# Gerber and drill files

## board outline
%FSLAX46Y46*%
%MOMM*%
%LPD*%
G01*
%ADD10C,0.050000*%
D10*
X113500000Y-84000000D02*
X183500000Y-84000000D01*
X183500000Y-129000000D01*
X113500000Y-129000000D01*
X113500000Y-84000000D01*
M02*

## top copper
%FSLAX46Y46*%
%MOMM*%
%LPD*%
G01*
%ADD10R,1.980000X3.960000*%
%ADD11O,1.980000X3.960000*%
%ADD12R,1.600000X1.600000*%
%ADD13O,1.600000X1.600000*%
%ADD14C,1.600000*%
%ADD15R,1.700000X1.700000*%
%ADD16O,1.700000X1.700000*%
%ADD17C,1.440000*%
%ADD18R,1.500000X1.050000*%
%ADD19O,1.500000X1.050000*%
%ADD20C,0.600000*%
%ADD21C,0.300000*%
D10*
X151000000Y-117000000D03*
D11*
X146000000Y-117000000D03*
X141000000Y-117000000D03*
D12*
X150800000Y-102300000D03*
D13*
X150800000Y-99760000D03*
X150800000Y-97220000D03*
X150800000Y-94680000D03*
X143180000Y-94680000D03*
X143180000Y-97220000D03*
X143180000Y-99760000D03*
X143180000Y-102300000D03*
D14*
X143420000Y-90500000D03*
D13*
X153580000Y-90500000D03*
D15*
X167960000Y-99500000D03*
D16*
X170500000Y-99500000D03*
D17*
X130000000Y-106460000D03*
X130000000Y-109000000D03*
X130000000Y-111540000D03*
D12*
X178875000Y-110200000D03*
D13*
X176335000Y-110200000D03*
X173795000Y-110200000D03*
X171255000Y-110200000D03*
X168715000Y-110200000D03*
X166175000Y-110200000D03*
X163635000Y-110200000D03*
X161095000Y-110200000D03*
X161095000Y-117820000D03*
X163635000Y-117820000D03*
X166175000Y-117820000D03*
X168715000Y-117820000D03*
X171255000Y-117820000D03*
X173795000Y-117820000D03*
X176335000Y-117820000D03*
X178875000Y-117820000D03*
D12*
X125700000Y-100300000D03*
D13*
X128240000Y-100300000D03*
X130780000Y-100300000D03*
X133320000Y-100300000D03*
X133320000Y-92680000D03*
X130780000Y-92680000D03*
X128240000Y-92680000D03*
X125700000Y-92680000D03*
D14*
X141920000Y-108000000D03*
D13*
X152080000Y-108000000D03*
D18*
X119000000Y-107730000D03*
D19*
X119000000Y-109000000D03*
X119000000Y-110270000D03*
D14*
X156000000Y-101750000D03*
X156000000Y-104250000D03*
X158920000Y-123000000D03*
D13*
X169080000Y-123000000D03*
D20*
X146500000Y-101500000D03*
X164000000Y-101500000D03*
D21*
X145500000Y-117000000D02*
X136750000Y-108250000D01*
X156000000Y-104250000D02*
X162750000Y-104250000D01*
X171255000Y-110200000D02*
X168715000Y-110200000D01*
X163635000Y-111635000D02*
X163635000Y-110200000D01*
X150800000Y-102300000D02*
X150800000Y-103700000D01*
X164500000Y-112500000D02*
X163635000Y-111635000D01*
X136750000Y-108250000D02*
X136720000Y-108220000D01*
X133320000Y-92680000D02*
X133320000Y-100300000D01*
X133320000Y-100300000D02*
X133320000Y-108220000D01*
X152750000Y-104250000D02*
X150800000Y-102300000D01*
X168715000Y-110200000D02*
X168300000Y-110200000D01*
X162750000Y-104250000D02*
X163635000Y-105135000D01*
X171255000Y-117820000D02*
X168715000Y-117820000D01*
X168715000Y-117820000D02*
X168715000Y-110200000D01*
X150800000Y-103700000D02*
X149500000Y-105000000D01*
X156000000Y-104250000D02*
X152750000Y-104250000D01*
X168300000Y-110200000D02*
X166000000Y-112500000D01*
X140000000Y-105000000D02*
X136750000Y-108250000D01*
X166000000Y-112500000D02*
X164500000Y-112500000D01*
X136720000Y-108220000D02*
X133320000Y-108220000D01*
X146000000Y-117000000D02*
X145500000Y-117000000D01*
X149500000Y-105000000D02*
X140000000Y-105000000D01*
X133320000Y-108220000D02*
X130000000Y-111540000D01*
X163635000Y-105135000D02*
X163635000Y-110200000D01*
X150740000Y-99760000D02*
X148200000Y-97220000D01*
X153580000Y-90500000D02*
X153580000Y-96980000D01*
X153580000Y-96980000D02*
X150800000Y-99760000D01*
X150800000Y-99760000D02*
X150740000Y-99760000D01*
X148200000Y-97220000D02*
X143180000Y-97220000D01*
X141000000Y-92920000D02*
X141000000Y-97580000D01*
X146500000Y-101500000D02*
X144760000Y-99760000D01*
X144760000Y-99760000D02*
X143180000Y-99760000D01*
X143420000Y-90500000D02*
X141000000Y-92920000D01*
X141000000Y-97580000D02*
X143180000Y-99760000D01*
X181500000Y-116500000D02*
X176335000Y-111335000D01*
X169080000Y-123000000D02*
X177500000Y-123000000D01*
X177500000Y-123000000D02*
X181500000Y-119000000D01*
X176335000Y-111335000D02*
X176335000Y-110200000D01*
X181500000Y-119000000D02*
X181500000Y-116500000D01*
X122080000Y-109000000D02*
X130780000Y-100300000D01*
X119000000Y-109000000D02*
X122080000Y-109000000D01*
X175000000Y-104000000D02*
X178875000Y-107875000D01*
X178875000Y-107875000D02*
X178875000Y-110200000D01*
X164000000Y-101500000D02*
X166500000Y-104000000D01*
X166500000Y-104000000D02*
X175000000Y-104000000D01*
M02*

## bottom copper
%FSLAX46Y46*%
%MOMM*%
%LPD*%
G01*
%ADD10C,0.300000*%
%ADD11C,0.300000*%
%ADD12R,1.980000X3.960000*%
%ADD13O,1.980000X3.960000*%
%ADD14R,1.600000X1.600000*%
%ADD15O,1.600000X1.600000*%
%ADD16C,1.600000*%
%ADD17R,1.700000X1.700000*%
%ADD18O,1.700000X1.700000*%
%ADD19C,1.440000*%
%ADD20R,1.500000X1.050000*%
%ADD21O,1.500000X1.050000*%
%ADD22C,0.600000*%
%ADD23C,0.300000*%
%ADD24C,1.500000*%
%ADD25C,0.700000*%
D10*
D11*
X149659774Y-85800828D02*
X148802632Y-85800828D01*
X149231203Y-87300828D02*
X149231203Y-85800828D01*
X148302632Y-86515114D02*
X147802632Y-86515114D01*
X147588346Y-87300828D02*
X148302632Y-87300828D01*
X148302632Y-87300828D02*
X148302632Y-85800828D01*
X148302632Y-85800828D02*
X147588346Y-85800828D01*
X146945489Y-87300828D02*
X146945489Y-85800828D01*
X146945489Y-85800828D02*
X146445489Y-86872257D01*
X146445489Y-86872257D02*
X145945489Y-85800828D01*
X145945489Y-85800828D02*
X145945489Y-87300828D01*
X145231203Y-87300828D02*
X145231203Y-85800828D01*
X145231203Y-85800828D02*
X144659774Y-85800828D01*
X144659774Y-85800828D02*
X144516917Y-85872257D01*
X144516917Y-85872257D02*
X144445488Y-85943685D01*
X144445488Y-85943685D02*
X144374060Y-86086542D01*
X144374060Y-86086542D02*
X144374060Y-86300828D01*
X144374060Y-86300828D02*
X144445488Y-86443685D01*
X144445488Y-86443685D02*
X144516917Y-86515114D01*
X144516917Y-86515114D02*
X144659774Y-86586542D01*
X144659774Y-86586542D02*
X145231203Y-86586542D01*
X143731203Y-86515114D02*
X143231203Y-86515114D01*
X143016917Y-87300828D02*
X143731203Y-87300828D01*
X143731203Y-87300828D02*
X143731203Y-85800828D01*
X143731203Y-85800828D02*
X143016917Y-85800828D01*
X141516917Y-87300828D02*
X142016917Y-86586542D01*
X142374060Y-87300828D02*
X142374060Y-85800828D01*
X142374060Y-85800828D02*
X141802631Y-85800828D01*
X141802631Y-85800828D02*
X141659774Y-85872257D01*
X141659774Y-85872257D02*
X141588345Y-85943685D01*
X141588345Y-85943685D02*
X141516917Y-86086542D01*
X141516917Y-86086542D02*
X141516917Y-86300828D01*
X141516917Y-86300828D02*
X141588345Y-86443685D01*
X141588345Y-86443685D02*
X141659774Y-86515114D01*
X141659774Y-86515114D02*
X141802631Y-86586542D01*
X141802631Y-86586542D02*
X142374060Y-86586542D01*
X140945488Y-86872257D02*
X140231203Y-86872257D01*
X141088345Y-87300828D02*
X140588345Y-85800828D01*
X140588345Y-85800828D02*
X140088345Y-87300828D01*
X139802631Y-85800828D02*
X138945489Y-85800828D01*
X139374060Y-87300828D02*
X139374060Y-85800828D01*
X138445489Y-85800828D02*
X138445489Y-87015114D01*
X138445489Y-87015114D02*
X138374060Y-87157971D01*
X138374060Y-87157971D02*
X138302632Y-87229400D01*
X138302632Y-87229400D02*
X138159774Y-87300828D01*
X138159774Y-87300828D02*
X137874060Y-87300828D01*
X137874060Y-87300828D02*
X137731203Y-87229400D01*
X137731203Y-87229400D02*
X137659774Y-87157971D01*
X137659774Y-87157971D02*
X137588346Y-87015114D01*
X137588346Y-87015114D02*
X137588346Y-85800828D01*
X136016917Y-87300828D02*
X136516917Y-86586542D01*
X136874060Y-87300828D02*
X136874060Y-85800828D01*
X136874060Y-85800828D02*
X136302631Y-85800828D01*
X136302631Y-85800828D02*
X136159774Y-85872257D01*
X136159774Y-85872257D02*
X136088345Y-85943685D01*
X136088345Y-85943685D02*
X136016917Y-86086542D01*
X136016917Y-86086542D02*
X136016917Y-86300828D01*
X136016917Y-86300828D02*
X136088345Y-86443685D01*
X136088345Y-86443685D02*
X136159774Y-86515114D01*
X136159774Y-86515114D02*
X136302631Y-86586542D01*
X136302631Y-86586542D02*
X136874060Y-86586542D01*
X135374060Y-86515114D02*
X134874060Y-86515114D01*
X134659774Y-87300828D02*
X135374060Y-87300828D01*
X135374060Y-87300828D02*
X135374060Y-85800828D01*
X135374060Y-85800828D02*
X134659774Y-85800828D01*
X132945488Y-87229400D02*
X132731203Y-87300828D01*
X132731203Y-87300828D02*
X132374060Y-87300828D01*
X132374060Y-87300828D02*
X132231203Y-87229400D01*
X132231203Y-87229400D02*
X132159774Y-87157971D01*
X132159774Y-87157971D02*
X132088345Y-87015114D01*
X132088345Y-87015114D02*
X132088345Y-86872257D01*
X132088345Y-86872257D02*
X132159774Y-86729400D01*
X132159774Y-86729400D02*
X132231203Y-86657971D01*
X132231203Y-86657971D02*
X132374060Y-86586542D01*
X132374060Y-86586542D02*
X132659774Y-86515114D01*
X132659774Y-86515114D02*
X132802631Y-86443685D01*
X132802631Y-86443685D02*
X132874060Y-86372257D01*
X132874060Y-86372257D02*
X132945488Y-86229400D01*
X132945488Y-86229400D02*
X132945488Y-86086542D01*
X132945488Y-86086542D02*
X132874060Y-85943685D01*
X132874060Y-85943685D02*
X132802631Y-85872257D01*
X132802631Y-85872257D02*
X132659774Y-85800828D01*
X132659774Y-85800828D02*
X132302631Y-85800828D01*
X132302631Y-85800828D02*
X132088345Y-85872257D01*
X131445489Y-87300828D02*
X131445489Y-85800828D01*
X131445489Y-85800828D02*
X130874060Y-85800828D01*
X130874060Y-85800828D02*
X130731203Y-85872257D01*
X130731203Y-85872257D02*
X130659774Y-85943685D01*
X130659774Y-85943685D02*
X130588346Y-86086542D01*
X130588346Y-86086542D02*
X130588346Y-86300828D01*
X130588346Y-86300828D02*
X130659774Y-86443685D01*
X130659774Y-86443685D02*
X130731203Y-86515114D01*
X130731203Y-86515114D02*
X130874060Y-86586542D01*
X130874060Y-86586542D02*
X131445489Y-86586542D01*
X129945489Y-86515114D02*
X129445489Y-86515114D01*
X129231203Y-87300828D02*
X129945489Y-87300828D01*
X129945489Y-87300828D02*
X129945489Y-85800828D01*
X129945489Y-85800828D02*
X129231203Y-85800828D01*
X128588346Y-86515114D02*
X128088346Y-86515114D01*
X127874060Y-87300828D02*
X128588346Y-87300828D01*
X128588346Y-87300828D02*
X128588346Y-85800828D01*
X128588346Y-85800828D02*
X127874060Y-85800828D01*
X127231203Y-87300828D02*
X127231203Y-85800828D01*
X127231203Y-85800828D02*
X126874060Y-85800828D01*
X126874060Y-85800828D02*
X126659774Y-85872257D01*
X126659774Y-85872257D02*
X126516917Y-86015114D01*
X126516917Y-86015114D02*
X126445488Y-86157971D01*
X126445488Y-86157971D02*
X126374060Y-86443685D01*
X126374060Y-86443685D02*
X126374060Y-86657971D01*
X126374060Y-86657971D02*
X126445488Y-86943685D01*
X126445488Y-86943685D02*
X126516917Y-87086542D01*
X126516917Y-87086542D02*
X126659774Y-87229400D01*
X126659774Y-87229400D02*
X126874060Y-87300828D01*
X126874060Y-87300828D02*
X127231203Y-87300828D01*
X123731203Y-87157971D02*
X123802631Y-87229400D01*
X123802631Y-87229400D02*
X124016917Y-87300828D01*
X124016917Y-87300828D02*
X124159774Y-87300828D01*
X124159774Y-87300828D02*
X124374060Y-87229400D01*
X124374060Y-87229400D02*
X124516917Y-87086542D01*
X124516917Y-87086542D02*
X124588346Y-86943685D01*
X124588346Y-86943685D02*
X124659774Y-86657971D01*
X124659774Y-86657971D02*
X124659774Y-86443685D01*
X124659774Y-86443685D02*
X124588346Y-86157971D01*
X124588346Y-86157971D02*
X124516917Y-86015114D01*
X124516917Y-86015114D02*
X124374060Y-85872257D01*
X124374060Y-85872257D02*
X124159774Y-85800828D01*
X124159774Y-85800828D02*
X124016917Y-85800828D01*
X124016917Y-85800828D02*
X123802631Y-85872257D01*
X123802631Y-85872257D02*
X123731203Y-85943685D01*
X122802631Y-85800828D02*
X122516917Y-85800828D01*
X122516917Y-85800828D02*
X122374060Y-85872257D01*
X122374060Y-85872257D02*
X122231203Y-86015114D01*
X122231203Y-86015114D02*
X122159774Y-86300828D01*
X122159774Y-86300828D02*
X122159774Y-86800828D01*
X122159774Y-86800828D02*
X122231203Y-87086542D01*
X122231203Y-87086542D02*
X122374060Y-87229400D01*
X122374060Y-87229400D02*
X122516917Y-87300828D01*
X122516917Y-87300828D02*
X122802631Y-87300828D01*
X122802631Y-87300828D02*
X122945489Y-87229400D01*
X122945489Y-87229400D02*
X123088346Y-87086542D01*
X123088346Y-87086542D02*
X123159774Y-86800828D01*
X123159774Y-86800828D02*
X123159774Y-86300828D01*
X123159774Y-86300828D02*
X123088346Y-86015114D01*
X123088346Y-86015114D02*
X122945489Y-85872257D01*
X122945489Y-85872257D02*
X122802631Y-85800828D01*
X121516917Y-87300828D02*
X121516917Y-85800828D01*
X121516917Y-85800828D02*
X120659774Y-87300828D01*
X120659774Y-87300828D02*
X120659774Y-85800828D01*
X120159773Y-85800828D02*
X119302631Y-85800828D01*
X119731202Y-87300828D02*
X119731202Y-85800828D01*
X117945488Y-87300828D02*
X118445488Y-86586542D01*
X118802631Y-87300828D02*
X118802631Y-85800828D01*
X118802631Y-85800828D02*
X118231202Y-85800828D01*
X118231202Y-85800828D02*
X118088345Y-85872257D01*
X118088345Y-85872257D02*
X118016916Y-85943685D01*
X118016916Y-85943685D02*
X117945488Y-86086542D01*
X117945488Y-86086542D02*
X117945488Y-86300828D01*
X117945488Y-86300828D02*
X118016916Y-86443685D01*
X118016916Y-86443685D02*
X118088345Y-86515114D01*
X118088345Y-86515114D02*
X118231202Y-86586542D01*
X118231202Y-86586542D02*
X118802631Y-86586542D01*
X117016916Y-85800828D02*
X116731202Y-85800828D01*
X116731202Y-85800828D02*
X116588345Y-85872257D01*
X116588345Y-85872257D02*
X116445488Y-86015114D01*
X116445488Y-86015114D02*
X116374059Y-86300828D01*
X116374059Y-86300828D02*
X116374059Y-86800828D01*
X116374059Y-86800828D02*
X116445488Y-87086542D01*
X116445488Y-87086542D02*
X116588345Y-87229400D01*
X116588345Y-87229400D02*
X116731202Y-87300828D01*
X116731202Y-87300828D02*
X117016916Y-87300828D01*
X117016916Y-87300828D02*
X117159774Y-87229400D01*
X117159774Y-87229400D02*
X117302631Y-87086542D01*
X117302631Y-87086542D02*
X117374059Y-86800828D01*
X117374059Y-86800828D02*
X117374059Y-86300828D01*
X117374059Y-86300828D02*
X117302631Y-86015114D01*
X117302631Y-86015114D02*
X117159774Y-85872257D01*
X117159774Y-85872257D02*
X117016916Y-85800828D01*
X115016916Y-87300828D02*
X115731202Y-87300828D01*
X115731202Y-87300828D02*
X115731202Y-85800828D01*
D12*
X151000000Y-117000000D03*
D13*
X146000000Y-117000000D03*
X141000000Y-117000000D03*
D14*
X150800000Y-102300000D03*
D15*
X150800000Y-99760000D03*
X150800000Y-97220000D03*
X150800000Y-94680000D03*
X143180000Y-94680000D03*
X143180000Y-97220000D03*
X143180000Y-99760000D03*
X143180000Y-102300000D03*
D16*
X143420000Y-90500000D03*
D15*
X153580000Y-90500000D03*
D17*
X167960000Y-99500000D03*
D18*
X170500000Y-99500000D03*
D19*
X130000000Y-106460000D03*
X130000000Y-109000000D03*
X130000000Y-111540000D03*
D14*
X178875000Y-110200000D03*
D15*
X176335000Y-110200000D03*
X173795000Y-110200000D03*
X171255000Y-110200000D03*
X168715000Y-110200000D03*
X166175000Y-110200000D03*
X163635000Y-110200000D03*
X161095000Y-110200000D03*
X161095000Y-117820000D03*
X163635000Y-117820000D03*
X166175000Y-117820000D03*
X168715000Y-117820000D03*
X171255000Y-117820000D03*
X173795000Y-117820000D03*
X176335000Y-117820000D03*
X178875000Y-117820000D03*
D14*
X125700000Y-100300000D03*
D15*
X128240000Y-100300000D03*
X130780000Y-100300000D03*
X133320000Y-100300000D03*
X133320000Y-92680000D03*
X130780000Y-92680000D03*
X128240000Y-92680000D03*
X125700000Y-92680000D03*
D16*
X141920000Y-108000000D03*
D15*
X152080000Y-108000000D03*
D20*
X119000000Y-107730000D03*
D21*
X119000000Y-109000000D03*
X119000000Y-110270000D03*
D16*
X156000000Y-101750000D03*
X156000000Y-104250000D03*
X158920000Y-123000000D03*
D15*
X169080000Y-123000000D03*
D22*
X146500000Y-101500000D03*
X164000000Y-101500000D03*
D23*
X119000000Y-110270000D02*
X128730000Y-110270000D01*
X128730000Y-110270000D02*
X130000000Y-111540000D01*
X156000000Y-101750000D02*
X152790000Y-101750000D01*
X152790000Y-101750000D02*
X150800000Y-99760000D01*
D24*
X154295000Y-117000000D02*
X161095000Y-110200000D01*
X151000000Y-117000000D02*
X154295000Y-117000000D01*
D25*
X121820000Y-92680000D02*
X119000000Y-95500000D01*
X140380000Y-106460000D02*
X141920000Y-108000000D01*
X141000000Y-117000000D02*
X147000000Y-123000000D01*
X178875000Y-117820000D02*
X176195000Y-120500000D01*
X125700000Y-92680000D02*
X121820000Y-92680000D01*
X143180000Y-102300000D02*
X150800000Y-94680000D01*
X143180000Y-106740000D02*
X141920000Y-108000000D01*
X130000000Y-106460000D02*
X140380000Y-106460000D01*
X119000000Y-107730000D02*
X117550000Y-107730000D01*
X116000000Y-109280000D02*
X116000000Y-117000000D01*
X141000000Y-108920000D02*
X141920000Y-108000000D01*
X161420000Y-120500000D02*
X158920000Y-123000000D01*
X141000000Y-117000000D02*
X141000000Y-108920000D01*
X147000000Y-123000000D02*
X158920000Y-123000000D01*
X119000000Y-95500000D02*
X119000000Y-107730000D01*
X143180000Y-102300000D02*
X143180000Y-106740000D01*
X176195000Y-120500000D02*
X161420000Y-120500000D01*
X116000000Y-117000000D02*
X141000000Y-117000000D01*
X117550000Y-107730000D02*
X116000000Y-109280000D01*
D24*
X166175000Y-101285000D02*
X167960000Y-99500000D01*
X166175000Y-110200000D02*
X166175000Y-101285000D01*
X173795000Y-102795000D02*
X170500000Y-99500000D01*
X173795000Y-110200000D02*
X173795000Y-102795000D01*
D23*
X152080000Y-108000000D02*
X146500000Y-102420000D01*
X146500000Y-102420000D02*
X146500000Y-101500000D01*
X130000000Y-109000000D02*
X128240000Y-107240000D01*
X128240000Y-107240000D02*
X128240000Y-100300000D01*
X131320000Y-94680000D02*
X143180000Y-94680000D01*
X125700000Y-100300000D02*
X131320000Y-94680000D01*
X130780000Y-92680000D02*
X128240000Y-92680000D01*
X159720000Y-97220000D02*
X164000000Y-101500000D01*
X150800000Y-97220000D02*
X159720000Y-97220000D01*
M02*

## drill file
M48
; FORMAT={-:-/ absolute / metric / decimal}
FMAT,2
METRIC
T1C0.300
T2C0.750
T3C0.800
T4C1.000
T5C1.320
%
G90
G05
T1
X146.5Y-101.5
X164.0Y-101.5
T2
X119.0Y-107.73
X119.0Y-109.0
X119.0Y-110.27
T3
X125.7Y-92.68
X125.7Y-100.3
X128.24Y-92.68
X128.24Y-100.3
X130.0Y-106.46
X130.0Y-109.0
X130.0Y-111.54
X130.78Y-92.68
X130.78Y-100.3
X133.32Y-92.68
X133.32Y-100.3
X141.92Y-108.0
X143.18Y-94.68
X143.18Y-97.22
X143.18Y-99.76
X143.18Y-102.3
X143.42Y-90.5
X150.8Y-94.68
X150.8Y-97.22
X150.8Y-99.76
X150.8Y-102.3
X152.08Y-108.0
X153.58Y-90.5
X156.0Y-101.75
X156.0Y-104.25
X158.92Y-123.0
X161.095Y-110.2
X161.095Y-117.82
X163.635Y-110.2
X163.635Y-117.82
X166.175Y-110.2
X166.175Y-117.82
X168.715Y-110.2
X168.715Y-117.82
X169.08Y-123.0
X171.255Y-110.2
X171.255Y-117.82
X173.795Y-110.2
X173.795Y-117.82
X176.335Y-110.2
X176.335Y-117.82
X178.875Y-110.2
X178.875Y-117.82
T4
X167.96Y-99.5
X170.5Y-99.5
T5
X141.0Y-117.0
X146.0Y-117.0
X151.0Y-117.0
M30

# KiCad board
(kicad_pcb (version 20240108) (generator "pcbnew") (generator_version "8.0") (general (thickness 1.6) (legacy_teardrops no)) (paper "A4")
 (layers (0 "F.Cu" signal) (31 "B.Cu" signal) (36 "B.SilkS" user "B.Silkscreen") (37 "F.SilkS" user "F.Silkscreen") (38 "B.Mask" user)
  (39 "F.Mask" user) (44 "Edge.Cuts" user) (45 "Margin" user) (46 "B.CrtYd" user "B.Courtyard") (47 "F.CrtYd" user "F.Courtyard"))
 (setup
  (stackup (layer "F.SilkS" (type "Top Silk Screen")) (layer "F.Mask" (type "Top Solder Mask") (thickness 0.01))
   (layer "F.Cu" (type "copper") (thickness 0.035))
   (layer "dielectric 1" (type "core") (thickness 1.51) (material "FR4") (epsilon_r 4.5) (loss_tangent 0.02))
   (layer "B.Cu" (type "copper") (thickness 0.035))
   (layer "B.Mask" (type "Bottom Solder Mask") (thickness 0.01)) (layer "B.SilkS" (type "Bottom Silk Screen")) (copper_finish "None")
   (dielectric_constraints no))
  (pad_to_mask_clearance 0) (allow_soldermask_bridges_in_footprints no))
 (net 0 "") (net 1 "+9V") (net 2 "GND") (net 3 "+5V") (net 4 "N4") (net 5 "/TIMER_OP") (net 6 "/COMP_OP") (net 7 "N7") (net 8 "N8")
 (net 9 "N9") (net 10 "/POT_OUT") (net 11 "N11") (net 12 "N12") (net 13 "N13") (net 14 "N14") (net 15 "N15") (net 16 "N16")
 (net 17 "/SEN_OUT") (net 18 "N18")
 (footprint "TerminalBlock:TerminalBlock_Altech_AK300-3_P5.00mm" (layer "F.Cu") (at 151 117 180)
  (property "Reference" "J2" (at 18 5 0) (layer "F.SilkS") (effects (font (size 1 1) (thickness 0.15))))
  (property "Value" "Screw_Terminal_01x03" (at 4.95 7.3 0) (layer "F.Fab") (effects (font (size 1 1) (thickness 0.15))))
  (pad "1" thru_hole rect (at 0 0 180) (size 1.98 3.96) (drill 1.32) (layers "*.Cu" "*.Mask") (remove_unused_layers no) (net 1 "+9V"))
  (pad "2" thru_hole oval (at 5 0 180) (size 1.98 3.96) (drill 1.32) (layers "*.Cu" "*.Mask") (remove_unused_layers no) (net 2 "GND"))
  (pad "3" thru_hole oval (at 10 0 180) (size 1.98 3.96) (drill 1.32) (layers "*.Cu" "*.Mask") (remove_unused_layers no) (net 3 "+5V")))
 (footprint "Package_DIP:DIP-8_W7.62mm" (layer "F.Cu") (at 150.8 102.3 180)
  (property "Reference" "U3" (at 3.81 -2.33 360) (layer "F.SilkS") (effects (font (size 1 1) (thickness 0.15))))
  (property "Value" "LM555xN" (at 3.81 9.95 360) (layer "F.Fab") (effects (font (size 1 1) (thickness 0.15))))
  (pad "1" thru_hole rect (at 0 0 180) (size 1.6 1.6) (drill 0.8) (layers "*.Cu" "*.Mask") (remove_unused_layers no) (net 2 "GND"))
  (pad "2" thru_hole oval (at 0 2.54 180) (size 1.6 1.6) (drill 0.8) (layers "*.Cu" "*.Mask") (remove_unused_layers no) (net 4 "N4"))
  (pad "3" thru_hole oval (at 0 5.08 180) (size 1.6 1.6) (drill 0.8) (layers "*.Cu" "*.Mask") (remove_unused_layers no) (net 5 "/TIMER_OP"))
  (pad "4" thru_hole oval (at 0 7.62 180) (size 1.6 1.6) (drill 0.8) (layers "*.Cu" "*.Mask") (remove_unused_layers no) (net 3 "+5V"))
  (pad "5" thru_hole oval (at 7.62 7.62 180) (size 1.6 1.6) (drill 0.8) (layers "*.Cu" "*.Mask") (remove_unused_layers no)
   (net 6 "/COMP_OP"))
  (pad "6" thru_hole oval (at 7.62 5.08 180) (size 1.6 1.6) (drill 0.8) (layers "*.Cu" "*.Mask") (remove_unused_layers no) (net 4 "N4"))
  (pad "7" thru_hole oval (at 7.62 2.54 180) (size 1.6 1.6) (drill 0.8) (layers "*.Cu" "*.Mask") (remove_unused_layers no) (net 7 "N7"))
  (pad "8" thru_hole oval (at 7.62 0 180) (size 1.6 1.6) (drill 0.8) (layers "*.Cu" "*.Mask") (remove_unused_layers no) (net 3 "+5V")))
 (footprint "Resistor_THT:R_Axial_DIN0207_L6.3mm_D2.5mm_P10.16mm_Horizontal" (layer "F.Cu") (at 143.42 90.5)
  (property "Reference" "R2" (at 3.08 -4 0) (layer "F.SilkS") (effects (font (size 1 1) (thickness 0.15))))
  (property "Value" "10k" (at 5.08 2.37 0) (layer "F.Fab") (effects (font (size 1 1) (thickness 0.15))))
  (pad "1" thru_hole circle (at 0 0) (size 1.6 1.6) (drill 0.8) (layers "*.Cu" "*.Mask") (remove_unused_layers no) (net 7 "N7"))
  (pad "2" thru_hole oval (at 10.16 0) (size 1.6 1.6) (drill 0.8) (layers "*.Cu" "*.Mask") (remove_unused_layers no) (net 4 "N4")))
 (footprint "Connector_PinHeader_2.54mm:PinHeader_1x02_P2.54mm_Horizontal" (layer "F.Cu") (at 167.96 99.5 90)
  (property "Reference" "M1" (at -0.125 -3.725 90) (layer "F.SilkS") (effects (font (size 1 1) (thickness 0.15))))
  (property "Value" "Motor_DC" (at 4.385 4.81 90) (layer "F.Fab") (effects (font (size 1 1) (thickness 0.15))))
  (pad "1" thru_hole rect (at 0 0 90) (size 1.7 1.7) (drill 1) (layers "*.Cu" "*.Mask") (remove_unused_layers no) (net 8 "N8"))
  (pad "2" thru_hole oval (at 0 2.54 90) (size 1.7 1.7) (drill 1) (layers "*.Cu" "*.Mask") (remove_unused_layers no) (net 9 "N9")))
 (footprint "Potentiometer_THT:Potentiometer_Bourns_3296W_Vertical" (layer "F.Cu") (at 130 106.46 90)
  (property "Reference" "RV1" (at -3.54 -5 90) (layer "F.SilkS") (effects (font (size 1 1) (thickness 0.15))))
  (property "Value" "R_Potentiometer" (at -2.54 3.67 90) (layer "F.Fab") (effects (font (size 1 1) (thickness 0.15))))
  (pad "1" thru_hole circle (at 0 0 90) (size 1.44 1.44) (drill 0.8) (layers "*.Cu" "*.Mask") (remove_unused_layers no) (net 3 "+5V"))
  (pad "2" thru_hole circle (at -2.54 0 90) (size 1.44 1.44) (drill 0.8) (layers "*.Cu" "*.Mask") (remove_unused_layers no)
   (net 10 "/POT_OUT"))
  (pad "3" thru_hole circle (at -5.08 0 90) (size 1.44 1.44) (drill 0.8) (layers "*.Cu" "*.Mask") (remove_unused_layers no) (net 2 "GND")))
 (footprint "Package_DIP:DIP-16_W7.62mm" (layer "F.Cu") (at 178.875 110.2 -90)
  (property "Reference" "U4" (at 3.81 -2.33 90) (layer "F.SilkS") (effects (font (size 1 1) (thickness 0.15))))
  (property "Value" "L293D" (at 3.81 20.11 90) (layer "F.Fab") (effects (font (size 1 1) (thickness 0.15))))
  (pad "1" thru_hole rect (at 0 0 270) (size 1.6 1.6) (drill 0.8) (layers "*.Cu" "*.Mask") (remove_unused_layers no) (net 5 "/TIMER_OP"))
  (pad "2" thru_hole oval (at 0 2.54 270) (size 1.6 1.6) (drill 0.8) (layers "*.Cu" "*.Mask") (remove_unused_layers no) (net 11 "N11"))
  (pad "3" thru_hole oval (at 0 5.08 270) (size 1.6 1.6) (drill 0.8) (layers "*.Cu" "*.Mask") (remove_unused_layers no) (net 9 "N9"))
  (pad "4" thru_hole oval (at 0 7.62 270) (size 1.6 1.6) (drill 0.8) (layers "*.Cu" "*.Mask") (remove_unused_layers no) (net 2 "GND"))
  (pad "5" thru_hole oval (at 0 10.16 270) (size 1.6 1.6) (drill 0.8) (layers "*.Cu" "*.Mask") (remove_unused_layers no) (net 2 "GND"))
  (pad "6" thru_hole oval (at 0 12.7 270) (size 1.6 1.6) (drill 0.8) (layers "*.Cu" "*.Mask") (remove_unused_layers no) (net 8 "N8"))
  (pad "7" thru_hole oval (at 0 15.24 270) (size 1.6 1.6) (drill 0.8) (layers "*.Cu" "*.Mask") (remove_unused_layers no) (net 2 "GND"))
  (pad "8" thru_hole oval (at 0 17.78 270) (size 1.6 1.6) (drill 0.8) (layers "*.Cu" "*.Mask") (remove_unused_layers no) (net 1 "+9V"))
  (pad "9" thru_hole oval (at 7.62 17.78 270) (size 1.6 1.6) (drill 0.8) (layers "*.Cu" "*.Mask") (remove_unused_layers no) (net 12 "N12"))
  (pad "10" thru_hole oval (at 7.62 15.24 270) (size 1.6 1.6) (drill 0.8) (layers "*.Cu" "*.Mask") (remove_unused_layers no) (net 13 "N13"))
  (pad "11" thru_hole oval (at 7.62 12.7 270) (size 1.6 1.6) (drill 0.8) (layers "*.Cu" "*.Mask") (remove_unused_layers no) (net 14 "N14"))
  (pad "12" thru_hole oval (at 7.62 10.16 270) (size 1.6 1.6) (drill 0.8) (layers "*.Cu" "*.Mask") (remove_unused_layers no) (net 2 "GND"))
  (pad "13" thru_hole oval (at 7.62 7.62 270) (size 1.6 1.6) (drill 0.8) (layers "*.Cu" "*.Mask") (remove_unused_layers no) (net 2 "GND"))
  (pad "14" thru_hole oval (at 7.62 5.08 270) (size 1.6 1.6) (drill 0.8) (layers "*.Cu" "*.Mask") (remove_unused_layers no) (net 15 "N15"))
  (pad "15" thru_hole oval (at 7.62 2.54 270) (size 1.6 1.6) (drill 0.8) (layers "*.Cu" "*.Mask") (remove_unused_layers no) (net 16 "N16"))
  (pad "16" thru_hole oval (at 7.62 0 270) (size 1.6 1.6) (drill 0.8) (layers "*.Cu" "*.Mask") (remove_unused_layers no) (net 3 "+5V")))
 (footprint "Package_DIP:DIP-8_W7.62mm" (layer "F.Cu") (at 125.7 100.3 90)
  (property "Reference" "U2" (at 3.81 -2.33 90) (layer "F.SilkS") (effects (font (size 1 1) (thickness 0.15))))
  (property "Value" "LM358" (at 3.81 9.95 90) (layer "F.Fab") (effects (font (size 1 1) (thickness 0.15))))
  (pad "1" thru_hole rect (at 0 0 90) (size 1.6 1.6) (drill 0.8) (layers "*.Cu" "*.Mask") (remove_unused_layers no) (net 6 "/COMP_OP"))
  (pad "2" thru_hole oval (at 0 2.54 90) (size 1.6 1.6) (drill 0.8) (layers "*.Cu" "*.Mask") (remove_unused_layers no) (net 10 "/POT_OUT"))
  (pad "3" thru_hole oval (at 0 5.08 90) (size 1.6 1.6) (drill 0.8) (layers "*.Cu" "*.Mask") (remove_unused_layers no) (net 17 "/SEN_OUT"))
  (pad "4" thru_hole oval (at 0 7.62 90) (size 1.6 1.6) (drill 0.8) (layers "*.Cu" "*.Mask") (remove_unused_layers no) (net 2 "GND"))
  (pad "5" thru_hole oval (at 7.62 7.62 90) (size 1.6 1.6) (drill 0.8) (layers "*.Cu" "*.Mask") (remove_unused_layers no) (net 2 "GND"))
  (pad "6" thru_hole oval (at 7.62 5.08 90) (size 1.6 1.6) (drill 0.8) (layers "*.Cu" "*.Mask") (remove_unused_layers no) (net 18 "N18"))
  (pad "7" thru_hole oval (at 7.62 2.54 90) (size 1.6 1.6) (drill 0.8) (layers "*.Cu" "*.Mask") (remove_unused_layers no) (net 18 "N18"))
  (pad "8" thru_hole oval (at 7.62 0 90) (size 1.6 1.6) (drill 0.8) (layers "*.Cu" "*.Mask") (remove_unused_layers no) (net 3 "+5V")))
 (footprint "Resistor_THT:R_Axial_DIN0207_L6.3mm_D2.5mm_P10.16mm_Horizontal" (layer "F.Cu") (at 141.92 108)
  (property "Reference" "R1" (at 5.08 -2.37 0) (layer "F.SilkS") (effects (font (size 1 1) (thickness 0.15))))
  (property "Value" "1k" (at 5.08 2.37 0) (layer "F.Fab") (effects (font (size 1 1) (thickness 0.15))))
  (pad "1" thru_hole circle (at 0 0) (size 1.6 1.6) (drill 0.8) (layers "*.Cu" "*.Mask") (remove_unused_layers no) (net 3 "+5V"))
  (pad "2" thru_hole oval (at 10.16 0) (size 1.6 1.6) (drill 0.8) (layers "*.Cu" "*.Mask") (remove_unused_layers no) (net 7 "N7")))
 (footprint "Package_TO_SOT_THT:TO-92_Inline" (layer "F.Cu") (at 119 107.73 -90)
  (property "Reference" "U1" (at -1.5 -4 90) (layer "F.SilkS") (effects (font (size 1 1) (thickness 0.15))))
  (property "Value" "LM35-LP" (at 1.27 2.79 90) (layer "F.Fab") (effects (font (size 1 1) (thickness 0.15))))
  (pad "1" thru_hole rect (at 0 0 270) (size 1.05 1.5) (drill 0.75) (layers "*.Cu" "*.Mask") (remove_unused_layers no) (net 3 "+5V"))
  (pad "2" thru_hole oval (at 1.27 0 270) (size 1.05 1.5) (drill 0.75) (layers "*.Cu" "*.Mask") (remove_unused_layers no)
   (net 17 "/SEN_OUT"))
  (pad "3" thru_hole oval (at 2.54 0 270) (size 1.05 1.5) (drill 0.75) (layers "*.Cu" "*.Mask") (remove_unused_layers no) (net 2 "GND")))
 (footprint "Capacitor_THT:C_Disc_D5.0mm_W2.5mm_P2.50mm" (layer "F.Cu") (at 156 101.75 -90)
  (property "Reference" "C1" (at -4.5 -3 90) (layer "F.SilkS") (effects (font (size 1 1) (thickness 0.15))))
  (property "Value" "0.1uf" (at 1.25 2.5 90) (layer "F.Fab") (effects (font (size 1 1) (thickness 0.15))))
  (pad "1" thru_hole circle (at 0 0 270) (size 1.6 1.6) (drill 0.8) (layers "*.Cu" "*.Mask") (remove_unused_layers no) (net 4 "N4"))
  (pad "2" thru_hole circle (at 2.5 0 270) (size 1.6 1.6) (drill 0.8) (layers "*.Cu" "*.Mask") (remove_unused_layers no) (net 2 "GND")))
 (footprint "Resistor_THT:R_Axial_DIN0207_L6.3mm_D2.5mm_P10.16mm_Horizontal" (layer "F.Cu") (at 158.92 123)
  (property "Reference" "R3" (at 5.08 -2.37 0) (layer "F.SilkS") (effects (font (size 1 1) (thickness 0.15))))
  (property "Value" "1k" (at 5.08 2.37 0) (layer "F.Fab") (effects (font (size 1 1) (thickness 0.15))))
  (pad "1" thru_hole circle (at 0 0) (size 1.6 1.6) (drill 0.8) (layers "*.Cu" "*.Mask") (remove_unused_layers no) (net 3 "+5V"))
  (pad "2" thru_hole oval (at 10.16 0) (size 1.6 1.6) (drill 0.8) (layers "*.Cu" "*.Mask") (remove_unused_layers no) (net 11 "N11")))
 (gr_rect (start 113.5 84) (end 183.5 129) (locked yes) (stroke (width 0.05) (type default)) (fill none) (layer "Edge.Cuts"))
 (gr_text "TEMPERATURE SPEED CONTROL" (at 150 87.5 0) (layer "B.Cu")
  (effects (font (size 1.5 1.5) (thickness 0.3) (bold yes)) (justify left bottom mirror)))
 (segment (start 145.5 117) (end 136.75 108.25) (width 0.3) (layer "F.Cu") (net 2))
 (segment (start 156 104.25) (end 162.75 104.25) (width 0.3) (layer "F.Cu") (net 2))
 (segment (start 171.255 110.2) (end 168.715 110.2) (width 0.3) (layer "F.Cu") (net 2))
 (segment (start 163.635 111.635) (end 163.635 110.2) (width 0.3) (layer "F.Cu") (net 2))
 (segment (start 150.8 102.3) (end 150.8 103.7) (width 0.3) (layer "F.Cu") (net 2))
 (segment (start 164.5 112.5) (end 163.635 111.635) (width 0.3) (layer "F.Cu") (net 2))
 (segment (start 136.75 108.25) (end 136.72 108.22) (width 0.3) (layer "F.Cu") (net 2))
 (segment (start 133.32 92.68) (end 133.32 100.3) (width 0.3) (layer "F.Cu") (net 2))
 (segment (start 133.32 100.3) (end 133.32 108.22) (width 0.3) (layer "F.Cu") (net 2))
 (segment (start 152.75 104.25) (end 150.8 102.3) (width 0.3) (layer "F.Cu") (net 2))
 (segment (start 168.715 110.2) (end 168.3 110.2) (width 0.3) (layer "F.Cu") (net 2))
 (segment (start 162.75 104.25) (end 163.635 105.135) (width 0.3) (layer "F.Cu") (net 2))
 (segment (start 171.255 117.82) (end 168.715 117.82) (width 0.3) (layer "F.Cu") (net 2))
 (segment (start 168.715 117.82) (end 168.715 110.2) (width 0.3) (layer "F.Cu") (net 2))
 (segment (start 150.8 103.7) (end 149.5 105) (width 0.3) (layer "F.Cu") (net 2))
 (segment (start 156 104.25) (end 152.75 104.25) (width 0.3) (layer "F.Cu") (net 2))
 (segment (start 168.3 110.2) (end 166 112.5) (width 0.3) (layer "F.Cu") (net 2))
 (segment (start 140 105) (end 136.75 108.25) (width 0.3) (layer "F.Cu") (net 2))
 (segment (start 166 112.5) (end 164.5 112.5) (width 0.3) (layer "F.Cu") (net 2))
 (segment (start 136.72 108.22) (end 133.32 108.22) (width 0.3) (layer "F.Cu") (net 2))
 (segment (start 146 117) (end 145.5 117) (width 0.3) (layer "F.Cu") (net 2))
 (segment (start 149.5 105) (end 140 105) (width 0.3) (layer "F.Cu") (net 2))
 (segment (start 133.32 108.22) (end 130 111.54) (width 0.3) (layer "F.Cu") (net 2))
 (segment (start 163.635 105.135) (end 163.635 110.2) (width 0.3) (layer "F.Cu") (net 2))
 (segment (start 119 110.27) (end 128.73 110.27) (width 0.3) (layer "B.Cu") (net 2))
 (segment (start 128.73 110.27) (end 130 111.54) (width 0.3) (layer "B.Cu") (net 2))
 (segment (start 150.74 99.76) (end 148.2 97.22) (width 0.3) (layer "F.Cu") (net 4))
 (segment (start 153.58 90.5) (end 153.58 96.98) (width 0.3) (layer "F.Cu") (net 4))
 (segment (start 153.58 96.98) (end 150.8 99.76) (width 0.3) (layer "F.Cu") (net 4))
 (segment (start 150.8 99.76) (end 150.74 99.76) (width 0.3) (layer "F.Cu") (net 4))
 (segment (start 148.2 97.22) (end 143.18 97.22) (width 0.3) (layer "F.Cu") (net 4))
 (segment (start 156 101.75) (end 152.79 101.75) (width 0.3) (layer "B.Cu") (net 4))
 (segment (start 152.79 101.75) (end 150.8 99.76) (width 0.3) (layer "B.Cu") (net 4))
 (segment (start 154.295 117) (end 161.095 110.2) (width 1.5) (layer "B.Cu") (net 1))
 (segment (start 151 117) (end 154.295 117) (width 1.5) (layer "B.Cu") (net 1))
 (segment (start 121.82 92.68) (end 119 95.5) (width 0.7) (layer "B.Cu") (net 3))
 (segment (start 140.38 106.46) (end 141.92 108) (width 0.7) (layer "B.Cu") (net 3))
 (segment (start 141 117) (end 147 123) (width 0.7) (layer "B.Cu") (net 3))
 (segment (start 178.875 117.82) (end 176.195 120.5) (width 0.7) (layer "B.Cu") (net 3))
 (segment (start 125.7 92.68) (end 121.82 92.68) (width 0.7) (layer "B.Cu") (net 3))
 (segment (start 143.18 102.3) (end 150.8 94.68) (width 0.7) (layer "B.Cu") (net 3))
 (segment (start 143.18 106.74) (end 141.92 108) (width 0.7) (layer "B.Cu") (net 3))
 (segment (start 130 106.46) (end 140.38 106.46) (width 0.7) (layer "B.Cu") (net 3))
 (segment (start 119 107.73) (end 117.55 107.73) (width 0.7) (layer "B.Cu") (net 3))
 (segment (start 116 109.28) (end 116 117) (width 0.7) (layer "B.Cu") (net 3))
 (segment (start 141 108.92) (end 141.92 108) (width 0.7) (layer "B.Cu") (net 3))
 (segment (start 161.42 120.5) (end 158.92 123) (width 0.7) (layer "B.Cu") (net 3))
 (segment (start 141 117) (end 141 108.92) (width 0.7) (layer "B.Cu") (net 3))
 (segment (start 147 123) (end 158.92 123) (width 0.7) (layer "B.Cu") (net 3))
 (segment (start 119 95.5) (end 119 107.73) (width 0.7) (layer "B.Cu") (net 3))
 (segment (start 143.18 102.3) (end 143.18 106.74) (width 0.7) (layer "B.Cu") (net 3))
 (segment (start 176.195 120.5) (end 161.42 120.5) (width 0.7) (layer "B.Cu") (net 3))
 (segment (start 116 117) (end 141 117) (width 0.7) (layer "B.Cu") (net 3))
 (segment (start 117.55 107.73) (end 116 109.28) (width 0.7) (layer "B.Cu") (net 3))
 (segment (start 166.175 101.285) (end 167.96 99.5) (width 1.5) (layer "B.Cu") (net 8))
 (segment (start 166.175 110.2) (end 166.175 101.285) (width 1.5) (layer "B.Cu") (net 8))
 (segment (start 173.795 102.795) (end 170.5 99.5) (width 1.5) (layer "B.Cu") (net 9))
 (segment (start 173.795 110.2) (end 173.795 102.795) (width 1.5) (layer "B.Cu") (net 9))
 (segment (start 141 92.92) (end 141 97.58) (width 0.3) (layer "F.Cu") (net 7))
 (segment (start 146.5 101.5) (end 144.76 99.76) (width 0.3) (layer "F.Cu") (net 7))
 (segment (start 144.76 99.76) (end 143.18 99.76) (width 0.3) (layer "F.Cu") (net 7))
 (segment (start 143.42 90.5) (end 141 92.92) (width 0.3) (layer "F.Cu") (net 7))
 (segment (start 141 97.58) (end 143.18 99.76) (width 0.3) (layer "F.Cu") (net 7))
 (via (at 146.5 101.5) (size 0.6) (drill 0.3) (layers "F.Cu" "B.Cu") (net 7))
 (segment (start 152.08 108) (end 146.5 102.42) (width 0.3) (layer "B.Cu") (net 7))
 (segment (start 146.5 102.42) (end 146.5 101.5) (width 0.3) (layer "B.Cu") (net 7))
 (segment (start 181.5 116.5) (end 176.335 111.335) (width 0.3) (layer "F.Cu") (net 11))
 (segment (start 169.08 123) (end 177.5 123) (width 0.3) (layer "F.Cu") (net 11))
 (segment (start 177.5 123) (end 181.5 119) (width 0.3) (layer "F.Cu") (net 11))
 (segment (start 176.335 111.335) (end 176.335 110.2) (width 0.3) (layer "F.Cu") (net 11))
 (segment (start 181.5 119) (end 181.5 116.5) (width 0.3) (layer "F.Cu") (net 11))
 (segment (start 130 109) (end 128.24 107.24) (width 0.3) (layer "B.Cu") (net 10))
 (segment (start 128.24 107.24) (end 128.24 100.3) (width 0.3) (layer "B.Cu") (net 10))
 (segment (start 122.08 109) (end 130.78 100.3) (width 0.3) (layer "F.Cu") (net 17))
 (segment (start 119 109) (end 122.08 109) (width 0.3) (layer "F.Cu") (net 17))
 (segment (start 131.32 94.68) (end 143.18 94.68) (width 0.3) (layer "B.Cu") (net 6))
 (segment (start 125.7 100.3) (end 131.32 94.68) (width 0.3) (layer "B.Cu") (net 6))
 (segment (start 130.78 92.68) (end 128.24 92.68) (width 0.3) (layer "B.Cu") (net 18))
 (segment (start 175 104) (end 178.875 107.875) (width 0.3) (layer "F.Cu") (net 5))
 (segment (start 178.875 107.875) (end 178.875 110.2) (width 0.3) (layer "F.Cu") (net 5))
 (segment (start 164 101.5) (end 166.5 104) (width 0.3) (layer "F.Cu") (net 5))
 (segment (start 166.5 104) (end 175 104) (width 0.3) (layer "F.Cu") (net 5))
 (via (at 164 101.5) (size 0.6) (drill 0.3) (layers "F.Cu" "B.Cu") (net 5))
 (segment (start 159.72 97.22) (end 164 101.5) (width 0.3) (layer "B.Cu") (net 5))
 (segment (start 150.8 97.22) (end 159.72 97.22) (width 0.3) (layer "B.Cu") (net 5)))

